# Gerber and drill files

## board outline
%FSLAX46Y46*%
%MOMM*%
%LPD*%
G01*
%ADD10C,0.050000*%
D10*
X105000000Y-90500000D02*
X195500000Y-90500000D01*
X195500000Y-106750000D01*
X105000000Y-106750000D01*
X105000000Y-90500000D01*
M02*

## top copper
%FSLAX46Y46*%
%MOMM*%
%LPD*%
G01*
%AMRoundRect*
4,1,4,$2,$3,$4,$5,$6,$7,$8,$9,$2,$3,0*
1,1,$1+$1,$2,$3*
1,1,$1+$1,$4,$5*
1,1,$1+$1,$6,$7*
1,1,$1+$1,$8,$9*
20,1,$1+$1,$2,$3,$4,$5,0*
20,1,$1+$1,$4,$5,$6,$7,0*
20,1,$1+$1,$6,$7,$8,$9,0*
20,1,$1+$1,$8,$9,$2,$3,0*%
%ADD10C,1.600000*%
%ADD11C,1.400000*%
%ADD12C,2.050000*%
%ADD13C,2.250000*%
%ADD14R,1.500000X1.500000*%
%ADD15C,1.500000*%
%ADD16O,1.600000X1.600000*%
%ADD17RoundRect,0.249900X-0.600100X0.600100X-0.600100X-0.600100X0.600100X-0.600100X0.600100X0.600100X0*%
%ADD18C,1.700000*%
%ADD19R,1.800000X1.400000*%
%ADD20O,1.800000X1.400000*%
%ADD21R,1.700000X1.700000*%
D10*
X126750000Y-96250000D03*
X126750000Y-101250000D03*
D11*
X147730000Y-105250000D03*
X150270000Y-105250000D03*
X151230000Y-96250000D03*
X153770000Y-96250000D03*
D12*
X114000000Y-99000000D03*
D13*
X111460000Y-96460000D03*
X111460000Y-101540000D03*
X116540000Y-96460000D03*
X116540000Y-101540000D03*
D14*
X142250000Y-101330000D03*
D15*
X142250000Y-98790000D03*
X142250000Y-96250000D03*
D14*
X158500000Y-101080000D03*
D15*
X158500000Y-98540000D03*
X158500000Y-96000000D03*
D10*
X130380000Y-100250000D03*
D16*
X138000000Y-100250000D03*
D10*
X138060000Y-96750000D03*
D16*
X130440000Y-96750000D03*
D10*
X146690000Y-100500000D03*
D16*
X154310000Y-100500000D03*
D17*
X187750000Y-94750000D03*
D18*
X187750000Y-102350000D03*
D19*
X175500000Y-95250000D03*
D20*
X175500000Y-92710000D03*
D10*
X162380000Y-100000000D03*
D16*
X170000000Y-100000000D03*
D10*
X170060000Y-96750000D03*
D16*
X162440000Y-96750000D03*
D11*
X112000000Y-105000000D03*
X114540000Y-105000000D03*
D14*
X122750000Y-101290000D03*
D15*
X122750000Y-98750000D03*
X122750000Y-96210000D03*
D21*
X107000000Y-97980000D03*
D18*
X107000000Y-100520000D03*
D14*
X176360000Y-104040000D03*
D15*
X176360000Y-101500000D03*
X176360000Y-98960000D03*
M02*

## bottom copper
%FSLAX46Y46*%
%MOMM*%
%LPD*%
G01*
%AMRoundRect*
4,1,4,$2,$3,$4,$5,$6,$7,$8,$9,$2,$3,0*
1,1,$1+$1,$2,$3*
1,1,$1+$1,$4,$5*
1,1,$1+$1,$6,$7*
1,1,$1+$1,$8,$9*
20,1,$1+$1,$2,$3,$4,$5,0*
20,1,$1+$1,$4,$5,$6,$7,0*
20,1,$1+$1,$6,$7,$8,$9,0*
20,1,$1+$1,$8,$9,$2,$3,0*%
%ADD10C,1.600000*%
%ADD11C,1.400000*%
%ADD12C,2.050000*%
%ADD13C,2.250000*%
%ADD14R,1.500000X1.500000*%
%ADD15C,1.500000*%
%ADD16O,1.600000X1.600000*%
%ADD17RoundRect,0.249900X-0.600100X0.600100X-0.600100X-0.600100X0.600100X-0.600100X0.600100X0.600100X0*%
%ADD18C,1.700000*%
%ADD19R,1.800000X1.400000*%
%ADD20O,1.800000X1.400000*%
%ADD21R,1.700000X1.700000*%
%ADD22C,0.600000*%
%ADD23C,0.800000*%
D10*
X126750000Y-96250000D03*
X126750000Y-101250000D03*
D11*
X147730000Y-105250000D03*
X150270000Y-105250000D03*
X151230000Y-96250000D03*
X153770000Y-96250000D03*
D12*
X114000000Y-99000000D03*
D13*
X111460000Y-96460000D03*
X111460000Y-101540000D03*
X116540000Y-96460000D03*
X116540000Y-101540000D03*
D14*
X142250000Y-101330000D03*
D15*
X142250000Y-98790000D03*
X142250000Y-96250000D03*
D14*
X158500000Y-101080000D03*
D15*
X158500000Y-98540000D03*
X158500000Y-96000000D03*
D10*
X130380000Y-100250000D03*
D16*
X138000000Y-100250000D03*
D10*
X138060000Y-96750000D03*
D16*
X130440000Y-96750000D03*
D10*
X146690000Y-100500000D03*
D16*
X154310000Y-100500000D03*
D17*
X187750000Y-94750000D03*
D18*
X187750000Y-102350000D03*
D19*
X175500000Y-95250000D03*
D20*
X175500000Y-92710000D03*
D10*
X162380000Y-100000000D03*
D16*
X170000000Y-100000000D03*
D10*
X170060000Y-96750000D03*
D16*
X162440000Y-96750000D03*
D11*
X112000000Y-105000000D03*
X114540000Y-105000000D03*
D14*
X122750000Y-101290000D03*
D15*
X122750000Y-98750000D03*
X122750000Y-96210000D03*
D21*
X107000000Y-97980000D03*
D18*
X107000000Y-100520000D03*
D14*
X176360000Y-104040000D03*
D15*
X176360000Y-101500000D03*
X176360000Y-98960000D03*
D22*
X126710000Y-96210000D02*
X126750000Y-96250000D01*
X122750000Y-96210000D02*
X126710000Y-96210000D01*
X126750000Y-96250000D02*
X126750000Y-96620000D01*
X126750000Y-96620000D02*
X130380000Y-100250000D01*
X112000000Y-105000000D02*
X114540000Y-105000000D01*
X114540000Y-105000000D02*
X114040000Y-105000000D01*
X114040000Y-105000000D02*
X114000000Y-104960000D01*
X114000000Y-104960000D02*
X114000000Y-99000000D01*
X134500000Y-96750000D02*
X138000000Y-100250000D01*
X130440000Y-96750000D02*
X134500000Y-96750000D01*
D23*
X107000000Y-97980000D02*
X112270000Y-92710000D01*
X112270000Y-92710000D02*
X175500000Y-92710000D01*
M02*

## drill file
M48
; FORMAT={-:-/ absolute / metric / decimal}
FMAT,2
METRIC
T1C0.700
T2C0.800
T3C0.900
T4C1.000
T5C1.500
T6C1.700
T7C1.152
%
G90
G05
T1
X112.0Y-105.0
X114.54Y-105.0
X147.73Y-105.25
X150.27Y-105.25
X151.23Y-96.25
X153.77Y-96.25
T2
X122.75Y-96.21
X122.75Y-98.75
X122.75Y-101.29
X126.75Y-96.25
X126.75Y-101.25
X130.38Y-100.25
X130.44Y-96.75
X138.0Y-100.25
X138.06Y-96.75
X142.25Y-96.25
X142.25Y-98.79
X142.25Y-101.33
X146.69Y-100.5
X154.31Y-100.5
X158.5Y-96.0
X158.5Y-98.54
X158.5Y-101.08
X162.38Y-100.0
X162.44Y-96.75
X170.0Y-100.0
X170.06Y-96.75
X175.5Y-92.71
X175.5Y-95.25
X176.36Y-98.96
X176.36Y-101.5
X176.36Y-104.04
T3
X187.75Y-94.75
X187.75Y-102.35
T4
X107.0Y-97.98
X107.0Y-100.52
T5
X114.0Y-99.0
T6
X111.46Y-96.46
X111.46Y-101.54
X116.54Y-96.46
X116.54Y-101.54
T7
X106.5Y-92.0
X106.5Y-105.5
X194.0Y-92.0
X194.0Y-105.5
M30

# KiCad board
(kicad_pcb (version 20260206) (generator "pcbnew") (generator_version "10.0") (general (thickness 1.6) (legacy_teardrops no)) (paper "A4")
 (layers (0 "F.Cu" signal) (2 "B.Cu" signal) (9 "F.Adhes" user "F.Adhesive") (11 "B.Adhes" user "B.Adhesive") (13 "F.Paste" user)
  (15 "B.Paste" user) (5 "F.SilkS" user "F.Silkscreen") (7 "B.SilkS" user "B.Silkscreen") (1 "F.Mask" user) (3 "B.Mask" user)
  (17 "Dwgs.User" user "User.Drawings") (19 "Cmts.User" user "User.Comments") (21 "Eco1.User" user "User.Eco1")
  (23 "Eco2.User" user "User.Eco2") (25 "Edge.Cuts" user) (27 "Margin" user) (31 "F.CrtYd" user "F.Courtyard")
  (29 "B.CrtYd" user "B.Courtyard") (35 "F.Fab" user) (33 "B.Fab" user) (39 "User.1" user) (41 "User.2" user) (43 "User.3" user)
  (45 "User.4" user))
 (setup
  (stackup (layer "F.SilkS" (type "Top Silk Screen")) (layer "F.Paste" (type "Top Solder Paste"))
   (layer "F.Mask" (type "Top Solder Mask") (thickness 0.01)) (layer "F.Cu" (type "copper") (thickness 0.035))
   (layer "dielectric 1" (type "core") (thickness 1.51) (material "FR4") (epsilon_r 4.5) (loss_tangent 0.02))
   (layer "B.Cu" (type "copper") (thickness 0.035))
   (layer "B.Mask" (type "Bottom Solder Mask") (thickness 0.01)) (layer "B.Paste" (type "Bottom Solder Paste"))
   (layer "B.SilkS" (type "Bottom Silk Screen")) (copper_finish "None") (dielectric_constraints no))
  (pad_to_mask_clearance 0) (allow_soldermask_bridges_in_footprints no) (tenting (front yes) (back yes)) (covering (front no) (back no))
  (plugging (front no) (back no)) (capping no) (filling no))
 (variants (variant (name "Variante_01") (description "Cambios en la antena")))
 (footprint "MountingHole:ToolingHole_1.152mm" (layer "F.Cu") (at 194 92)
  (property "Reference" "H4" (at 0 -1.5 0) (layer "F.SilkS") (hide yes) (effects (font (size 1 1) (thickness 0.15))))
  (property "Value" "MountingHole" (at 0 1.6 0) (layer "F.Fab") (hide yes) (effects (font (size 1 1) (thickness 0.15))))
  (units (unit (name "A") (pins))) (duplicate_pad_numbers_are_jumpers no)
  (pad "" np_thru_hole circle (at 0 0) (size 1.152 1.152) (drill 1.152) (layers "*.Cu" "*.Mask") (solder_mask_margin 0.074))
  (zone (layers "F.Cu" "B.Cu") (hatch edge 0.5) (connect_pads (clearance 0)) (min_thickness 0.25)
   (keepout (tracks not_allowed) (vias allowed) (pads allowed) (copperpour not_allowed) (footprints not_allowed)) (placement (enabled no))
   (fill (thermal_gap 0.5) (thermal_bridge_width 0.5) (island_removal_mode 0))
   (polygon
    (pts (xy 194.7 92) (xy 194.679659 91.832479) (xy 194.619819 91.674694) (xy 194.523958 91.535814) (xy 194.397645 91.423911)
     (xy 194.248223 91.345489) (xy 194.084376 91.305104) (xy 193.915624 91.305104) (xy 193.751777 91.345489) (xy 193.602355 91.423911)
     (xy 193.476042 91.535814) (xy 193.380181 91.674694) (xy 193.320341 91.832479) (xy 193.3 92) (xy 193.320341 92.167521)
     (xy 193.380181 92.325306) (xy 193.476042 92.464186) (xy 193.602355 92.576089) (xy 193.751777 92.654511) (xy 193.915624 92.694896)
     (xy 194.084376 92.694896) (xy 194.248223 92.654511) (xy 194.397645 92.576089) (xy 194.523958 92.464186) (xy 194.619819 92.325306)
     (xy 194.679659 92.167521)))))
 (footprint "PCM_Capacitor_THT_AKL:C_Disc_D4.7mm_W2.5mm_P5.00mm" (layer "F.Cu") (at 126.75 96.25 -90)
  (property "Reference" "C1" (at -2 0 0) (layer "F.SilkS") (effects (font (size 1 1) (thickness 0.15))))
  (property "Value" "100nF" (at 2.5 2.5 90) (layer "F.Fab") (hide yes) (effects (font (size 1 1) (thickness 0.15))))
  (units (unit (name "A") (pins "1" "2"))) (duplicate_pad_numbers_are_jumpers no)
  (pad "1" thru_hole circle (at 0 0 270) (size 1.6 1.6) (drill 0.8) (layers "*.Cu" "*.Mask") (remove_unused_layers no) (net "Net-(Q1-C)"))
  (pad "2" thru_hole circle (at 5 0 270) (size 1.6 1.6) (drill 0.8) (layers "*.Cu" "*.Mask") (remove_unused_layers no) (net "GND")))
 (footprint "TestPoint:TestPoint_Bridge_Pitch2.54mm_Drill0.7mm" (layer "F.Cu") (at 147.73 105.25)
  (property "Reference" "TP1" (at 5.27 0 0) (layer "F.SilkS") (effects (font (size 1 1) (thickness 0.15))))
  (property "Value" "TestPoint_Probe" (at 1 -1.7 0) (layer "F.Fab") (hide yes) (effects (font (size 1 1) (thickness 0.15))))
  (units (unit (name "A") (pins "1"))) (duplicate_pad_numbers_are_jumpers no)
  (pad "1" thru_hole circle (at 0 0) (size 1.4 1.4) (drill 0.7) (layers "*.Cu" "*.Mask") (remove_unused_layers no) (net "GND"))
  (pad "1" thru_hole circle (at 2.54 0) (size 1.4 1.4) (drill 0.7) (layers "*.Cu" "*.Mask") (remove_unused_layers no) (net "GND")))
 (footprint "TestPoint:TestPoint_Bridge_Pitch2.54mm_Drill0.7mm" (layer "F.Cu") (at 151.23 96.25)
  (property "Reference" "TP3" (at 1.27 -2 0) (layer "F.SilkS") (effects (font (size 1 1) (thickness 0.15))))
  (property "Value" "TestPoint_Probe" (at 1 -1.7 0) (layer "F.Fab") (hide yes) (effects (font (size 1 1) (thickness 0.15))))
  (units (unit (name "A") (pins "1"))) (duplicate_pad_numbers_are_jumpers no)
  (pad "1" thru_hole circle (at 0 0) (size 1.4 1.4) (drill 0.7) (layers "*.Cu" "*.Mask") (remove_unused_layers no) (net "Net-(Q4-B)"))
  (pad "1" thru_hole circle (at 2.54 0) (size 1.4 1.4) (drill 0.7) (layers "*.Cu" "*.Mask") (remove_unused_layers no) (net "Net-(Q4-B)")))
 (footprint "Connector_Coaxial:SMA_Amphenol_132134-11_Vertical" (layer "F.Cu") (at 114 99)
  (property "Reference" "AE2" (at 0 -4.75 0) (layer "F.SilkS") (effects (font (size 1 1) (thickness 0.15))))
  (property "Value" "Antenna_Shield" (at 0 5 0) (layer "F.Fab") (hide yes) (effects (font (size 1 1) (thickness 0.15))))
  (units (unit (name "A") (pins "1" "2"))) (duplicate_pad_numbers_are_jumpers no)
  (pad "1" thru_hole circle (at 0 0) (size 2.05 2.05) (drill 1.5) (layers "*.Cu" "*.Mask") (remove_unused_layers no) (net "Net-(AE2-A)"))
  (pad "2" thru_hole circle (at -2.54 -2.54) (size 2.25 2.25) (drill 1.7) (layers "*.Cu" "*.Mask") (remove_unused_layers no) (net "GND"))
  (pad "2" thru_hole circle (at -2.54 2.54) (size 2.25 2.25) (drill 1.7) (layers "*.Cu" "*.Mask") (remove_unused_layers no) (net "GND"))
  (pad "2" thru_hole circle (at 2.54 -2.54) (size 2.25 2.25) (drill 1.7) (layers "*.Cu" "*.Mask") (remove_unused_layers no) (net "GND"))
  (pad "2" thru_hole circle (at 2.54 2.54) (size 2.25 2.25) (drill 1.7) (layers "*.Cu" "*.Mask") (remove_unused_layers no) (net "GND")))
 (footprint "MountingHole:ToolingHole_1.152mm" (layer "F.Cu") (at 194 105.5)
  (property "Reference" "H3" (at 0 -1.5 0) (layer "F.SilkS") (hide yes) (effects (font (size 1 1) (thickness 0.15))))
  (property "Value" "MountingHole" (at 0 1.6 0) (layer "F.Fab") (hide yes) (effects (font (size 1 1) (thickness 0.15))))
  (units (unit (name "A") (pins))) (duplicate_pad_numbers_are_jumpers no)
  (pad "" np_thru_hole circle (at 0 0) (size 1.152 1.152) (drill 1.152) (layers "*.Cu" "*.Mask") (solder_mask_margin 0.074))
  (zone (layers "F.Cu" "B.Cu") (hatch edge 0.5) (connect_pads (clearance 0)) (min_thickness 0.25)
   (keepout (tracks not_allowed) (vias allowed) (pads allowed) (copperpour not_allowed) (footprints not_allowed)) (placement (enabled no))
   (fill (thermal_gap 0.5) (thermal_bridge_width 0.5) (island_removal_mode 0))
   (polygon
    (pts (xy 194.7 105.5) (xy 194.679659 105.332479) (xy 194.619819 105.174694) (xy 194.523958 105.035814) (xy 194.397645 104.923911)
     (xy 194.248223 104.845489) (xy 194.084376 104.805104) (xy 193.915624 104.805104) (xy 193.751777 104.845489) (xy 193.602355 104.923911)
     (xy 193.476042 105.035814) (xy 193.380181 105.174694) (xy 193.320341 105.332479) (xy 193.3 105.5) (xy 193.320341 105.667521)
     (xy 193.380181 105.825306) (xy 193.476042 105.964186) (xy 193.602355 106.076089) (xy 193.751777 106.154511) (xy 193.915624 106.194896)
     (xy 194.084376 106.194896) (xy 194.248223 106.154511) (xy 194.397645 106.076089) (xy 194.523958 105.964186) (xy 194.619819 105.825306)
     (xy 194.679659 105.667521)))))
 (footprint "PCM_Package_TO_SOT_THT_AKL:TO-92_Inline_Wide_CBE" (layer "F.Cu") (at 142.25 101.33 90)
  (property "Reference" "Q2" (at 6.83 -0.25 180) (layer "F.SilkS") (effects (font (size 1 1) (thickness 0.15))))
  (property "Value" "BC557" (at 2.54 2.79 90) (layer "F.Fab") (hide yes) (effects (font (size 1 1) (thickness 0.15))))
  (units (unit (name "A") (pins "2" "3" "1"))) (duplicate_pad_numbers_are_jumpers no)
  (pad "1" thru_hole rect (at 0 0 180) (size 1.5 1.5) (drill 0.8) (layers "*.Cu" "*.Mask") (remove_unused_layers no) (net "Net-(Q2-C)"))
  (pad "2" thru_hole circle (at 2.54 0 180) (size 1.5 1.5) (drill 0.8) (layers "*.Cu" "*.Mask") (remove_unused_layers no) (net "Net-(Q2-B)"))
  (pad "3" thru_hole circle (at 5.08 0 180) (size 1.5 1.5) (drill 0.8) (layers "*.Cu" "*.Mask") (remove_unused_layers no) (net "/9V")))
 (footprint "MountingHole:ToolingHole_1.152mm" (layer "F.Cu") (at 106.5 92)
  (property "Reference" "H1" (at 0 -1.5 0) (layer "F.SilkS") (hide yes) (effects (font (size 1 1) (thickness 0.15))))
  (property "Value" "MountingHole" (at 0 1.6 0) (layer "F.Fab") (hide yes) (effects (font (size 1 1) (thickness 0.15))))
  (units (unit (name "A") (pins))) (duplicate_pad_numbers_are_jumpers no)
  (pad "" np_thru_hole circle (at 0 0) (size 1.152 1.152) (drill 1.152) (layers "*.Cu" "*.Mask") (solder_mask_margin 0.074))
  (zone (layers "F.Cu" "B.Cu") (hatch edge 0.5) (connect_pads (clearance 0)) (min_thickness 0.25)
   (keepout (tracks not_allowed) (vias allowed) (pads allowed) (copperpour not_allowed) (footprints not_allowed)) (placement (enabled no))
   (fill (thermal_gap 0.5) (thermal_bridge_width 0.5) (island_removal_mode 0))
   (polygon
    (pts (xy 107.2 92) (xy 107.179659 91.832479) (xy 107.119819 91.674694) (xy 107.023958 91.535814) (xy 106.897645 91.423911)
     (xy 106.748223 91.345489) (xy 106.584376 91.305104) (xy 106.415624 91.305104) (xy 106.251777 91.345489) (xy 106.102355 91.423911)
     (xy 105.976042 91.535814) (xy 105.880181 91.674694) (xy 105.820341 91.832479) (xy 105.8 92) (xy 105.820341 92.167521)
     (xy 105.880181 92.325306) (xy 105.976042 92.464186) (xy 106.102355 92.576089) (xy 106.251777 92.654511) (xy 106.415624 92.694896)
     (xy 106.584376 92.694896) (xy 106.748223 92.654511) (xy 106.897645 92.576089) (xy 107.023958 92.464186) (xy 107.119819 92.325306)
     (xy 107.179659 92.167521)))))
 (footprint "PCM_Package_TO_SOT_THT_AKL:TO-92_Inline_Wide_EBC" (layer "F.Cu") (at 158.5 101.08 90)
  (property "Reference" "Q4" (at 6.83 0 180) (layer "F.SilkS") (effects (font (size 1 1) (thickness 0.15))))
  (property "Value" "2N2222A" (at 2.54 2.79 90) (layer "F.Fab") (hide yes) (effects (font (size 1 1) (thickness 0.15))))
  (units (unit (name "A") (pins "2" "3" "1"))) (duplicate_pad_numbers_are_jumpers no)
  (pad "1" thru_hole rect (at 0 0 180) (size 1.5 1.5) (drill 0.8) (layers "*.Cu" "*.Mask") (remove_unused_layers no) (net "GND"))
  (pad "2" thru_hole circle (at 2.54 0 180) (size 1.5 1.5) (drill 0.8) (layers "*.Cu" "*.Mask") (remove_unused_layers no) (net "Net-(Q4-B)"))
  (pad "3" thru_hole circle (at 5.08 0 180) (size 1.5 1.5) (drill 0.8) (layers "*.Cu" "*.Mask") (remove_unused_layers no) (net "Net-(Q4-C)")))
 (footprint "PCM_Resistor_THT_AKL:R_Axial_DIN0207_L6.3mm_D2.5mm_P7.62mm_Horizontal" (layer "F.Cu") (at 130.38 100.25)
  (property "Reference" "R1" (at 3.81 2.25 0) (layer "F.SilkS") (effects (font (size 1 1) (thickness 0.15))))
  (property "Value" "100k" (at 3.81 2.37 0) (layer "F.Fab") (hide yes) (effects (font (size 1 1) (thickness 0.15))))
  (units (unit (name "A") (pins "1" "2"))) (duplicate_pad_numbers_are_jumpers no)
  (pad "1" thru_hole circle (at 0 0) (size 1.6 1.6) (drill 0.8) (layers "*.Cu" "*.Mask") (remove_unused_layers no) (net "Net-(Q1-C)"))
  (pad "2" thru_hole oval (at 7.62 0) (size 1.6 1.6) (drill 0.8) (layers "*.Cu" "*.Mask") (remove_unused_layers no) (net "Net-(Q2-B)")))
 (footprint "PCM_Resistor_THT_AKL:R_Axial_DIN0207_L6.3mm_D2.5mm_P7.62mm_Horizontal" (layer "F.Cu") (at 138.06 96.75 180)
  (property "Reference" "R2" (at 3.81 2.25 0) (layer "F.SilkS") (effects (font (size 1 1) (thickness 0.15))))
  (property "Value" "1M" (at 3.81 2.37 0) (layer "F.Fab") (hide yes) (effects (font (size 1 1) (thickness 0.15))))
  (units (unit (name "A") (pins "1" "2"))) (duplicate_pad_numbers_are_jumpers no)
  (pad "1" thru_hole circle (at 0 0 180) (size 1.6 1.6) (drill 0.8) (layers "*.Cu" "*.Mask") (remove_unused_layers no) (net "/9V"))
  (pad "2" thru_hole oval (at 7.62 0 180) (size 1.6 1.6) (drill 0.8) (layers "*.Cu" "*.Mask") (remove_unused_layers no) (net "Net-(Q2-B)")))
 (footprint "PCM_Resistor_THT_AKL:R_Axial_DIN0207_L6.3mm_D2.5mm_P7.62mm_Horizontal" (layer "F.Cu") (at 146.69 100.5)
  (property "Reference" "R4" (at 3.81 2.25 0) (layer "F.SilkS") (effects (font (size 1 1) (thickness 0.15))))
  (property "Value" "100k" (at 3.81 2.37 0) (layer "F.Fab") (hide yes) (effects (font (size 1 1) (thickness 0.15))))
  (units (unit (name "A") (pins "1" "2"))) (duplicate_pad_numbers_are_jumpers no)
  (pad "1" thru_hole circle (at 0 0) (size 1.6 1.6) (drill 0.8) (layers "*.Cu" "*.Mask") (remove_unused_layers no) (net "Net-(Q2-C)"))
  (pad "2" thru_hole oval (at 7.62 0) (size 1.6 1.6) (drill 0.8) (layers "*.Cu" "*.Mask") (remove_unused_layers no) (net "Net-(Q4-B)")))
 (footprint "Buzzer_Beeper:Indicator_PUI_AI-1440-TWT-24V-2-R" (layer "F.Cu") (at 187.75 94.75 -90)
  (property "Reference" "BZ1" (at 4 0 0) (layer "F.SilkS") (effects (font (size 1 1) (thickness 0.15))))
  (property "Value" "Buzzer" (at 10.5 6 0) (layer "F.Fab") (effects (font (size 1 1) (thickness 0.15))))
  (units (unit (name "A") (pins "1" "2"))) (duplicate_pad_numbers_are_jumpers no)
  (pad "1" thru_hole roundrect (at 0 0 270) (size 1.7 1.7) (drill 0.9) (layers "*.Cu" "*.Mask") (remove_unused_layers no)
   (roundrect_rratio 0.147) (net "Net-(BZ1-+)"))
  (pad "2" thru_hole circle (at 7.6 0 270) (size 1.7 1.7) (drill 0.9) (layers "*.Cu" "*.Mask") (remove_unused_layers no) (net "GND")))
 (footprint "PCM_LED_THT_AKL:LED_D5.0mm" (layer "F.Cu") (at 175.5 95.25 90)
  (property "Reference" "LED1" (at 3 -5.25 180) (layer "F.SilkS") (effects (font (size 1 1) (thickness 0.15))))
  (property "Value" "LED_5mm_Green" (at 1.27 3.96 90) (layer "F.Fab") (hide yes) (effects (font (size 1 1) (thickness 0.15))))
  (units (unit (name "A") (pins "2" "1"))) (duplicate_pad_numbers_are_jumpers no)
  (pad "1" thru_hole rect (at 0 0 90) (size 1.4 1.8) (drill 0.8) (layers "*.Cu" "*.Mask") (remove_unused_layers no) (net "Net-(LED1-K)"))
  (pad "2" thru_hole oval (at 2.54 0 90) (size 1.4 1.8) (drill 0.8) (layers "*.Cu" "*.Mask") (remove_unused_layers no) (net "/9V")))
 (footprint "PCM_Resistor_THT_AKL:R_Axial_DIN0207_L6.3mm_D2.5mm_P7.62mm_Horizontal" (layer "F.Cu") (at 162.38 100)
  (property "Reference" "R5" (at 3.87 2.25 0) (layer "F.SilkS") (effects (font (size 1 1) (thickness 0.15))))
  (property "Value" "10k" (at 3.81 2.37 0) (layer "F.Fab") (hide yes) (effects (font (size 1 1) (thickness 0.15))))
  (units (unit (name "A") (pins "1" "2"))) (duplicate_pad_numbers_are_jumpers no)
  (pad "1" thru_hole circle (at 0 0) (size 1.6 1.6) (drill 0.8) (layers "*.Cu" "*.Mask") (remove_unused_layers no) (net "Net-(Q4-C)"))
  (pad "2" thru_hole oval (at 7.62 0) (size 1.6 1.6) (drill 0.8) (layers "*.Cu" "*.Mask") (remove_unused_layers no) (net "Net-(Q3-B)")))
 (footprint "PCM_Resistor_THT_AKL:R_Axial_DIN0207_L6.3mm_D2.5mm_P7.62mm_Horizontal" (layer "F.Cu") (at 170.06 96.75 180)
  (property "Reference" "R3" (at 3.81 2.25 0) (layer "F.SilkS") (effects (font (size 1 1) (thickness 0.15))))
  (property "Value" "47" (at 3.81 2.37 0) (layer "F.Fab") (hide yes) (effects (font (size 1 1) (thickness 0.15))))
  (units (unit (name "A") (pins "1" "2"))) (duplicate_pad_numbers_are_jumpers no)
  (pad "1" thru_hole circle (at 0 0 180) (size 1.6 1.6) (drill 0.8) (layers "*.Cu" "*.Mask") (remove_unused_layers no) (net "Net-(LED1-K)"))
  (pad "2" thru_hole oval (at 7.62 0 180) (size 1.6 1.6) (drill 0.8) (layers "*.Cu" "*.Mask") (remove_unused_layers no) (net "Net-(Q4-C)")))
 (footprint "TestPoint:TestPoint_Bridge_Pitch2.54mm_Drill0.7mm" (layer "F.Cu") (at 112 105)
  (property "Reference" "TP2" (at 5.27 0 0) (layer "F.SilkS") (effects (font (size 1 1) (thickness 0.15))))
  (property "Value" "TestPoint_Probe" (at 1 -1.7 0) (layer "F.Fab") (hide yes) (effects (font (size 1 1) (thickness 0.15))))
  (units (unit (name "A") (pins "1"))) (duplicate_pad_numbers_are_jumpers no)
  (pad "1" thru_hole circle (at 0 0) (size 1.4 1.4) (drill 0.7) (layers "*.Cu" "*.Mask") (remove_unused_layers no) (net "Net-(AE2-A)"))
  (pad "1" thru_hole circle (at 2.54 0) (size 1.4 1.4) (drill 0.7) (layers "*.Cu" "*.Mask") (remove_unused_layers no) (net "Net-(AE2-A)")))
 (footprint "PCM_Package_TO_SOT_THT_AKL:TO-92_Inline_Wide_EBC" (layer "F.Cu") (at 122.75 101.29 90)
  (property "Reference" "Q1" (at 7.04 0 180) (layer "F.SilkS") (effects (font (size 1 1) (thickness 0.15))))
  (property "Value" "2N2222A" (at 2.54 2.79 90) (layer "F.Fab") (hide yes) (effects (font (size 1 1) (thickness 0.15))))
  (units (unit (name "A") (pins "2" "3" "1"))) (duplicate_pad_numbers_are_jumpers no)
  (pad "1" thru_hole rect (at 0 0 180) (size 1.5 1.5) (drill 0.8) (layers "*.Cu" "*.Mask") (remove_unused_layers no) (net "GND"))
  (pad "2" thru_hole circle (at 2.54 0 180) (size 1.5 1.5) (drill 0.8) (layers "*.Cu" "*.Mask") (remove_unused_layers no)
   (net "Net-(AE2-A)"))
  (pad "3" thru_hole circle (at 5.08 0 180) (size 1.5 1.5) (drill 0.8) (layers "*.Cu" "*.Mask") (remove_unused_layers no) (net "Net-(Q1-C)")))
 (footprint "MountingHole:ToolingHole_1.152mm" (layer "F.Cu") (at 106.5 105.5)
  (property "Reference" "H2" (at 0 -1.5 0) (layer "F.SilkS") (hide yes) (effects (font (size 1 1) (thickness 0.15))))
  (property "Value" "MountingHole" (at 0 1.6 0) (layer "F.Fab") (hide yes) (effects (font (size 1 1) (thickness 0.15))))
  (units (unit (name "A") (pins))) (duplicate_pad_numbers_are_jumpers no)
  (pad "" np_thru_hole circle (at 0 0) (size 1.152 1.152) (drill 1.152) (layers "*.Cu" "*.Mask") (solder_mask_margin 0.074))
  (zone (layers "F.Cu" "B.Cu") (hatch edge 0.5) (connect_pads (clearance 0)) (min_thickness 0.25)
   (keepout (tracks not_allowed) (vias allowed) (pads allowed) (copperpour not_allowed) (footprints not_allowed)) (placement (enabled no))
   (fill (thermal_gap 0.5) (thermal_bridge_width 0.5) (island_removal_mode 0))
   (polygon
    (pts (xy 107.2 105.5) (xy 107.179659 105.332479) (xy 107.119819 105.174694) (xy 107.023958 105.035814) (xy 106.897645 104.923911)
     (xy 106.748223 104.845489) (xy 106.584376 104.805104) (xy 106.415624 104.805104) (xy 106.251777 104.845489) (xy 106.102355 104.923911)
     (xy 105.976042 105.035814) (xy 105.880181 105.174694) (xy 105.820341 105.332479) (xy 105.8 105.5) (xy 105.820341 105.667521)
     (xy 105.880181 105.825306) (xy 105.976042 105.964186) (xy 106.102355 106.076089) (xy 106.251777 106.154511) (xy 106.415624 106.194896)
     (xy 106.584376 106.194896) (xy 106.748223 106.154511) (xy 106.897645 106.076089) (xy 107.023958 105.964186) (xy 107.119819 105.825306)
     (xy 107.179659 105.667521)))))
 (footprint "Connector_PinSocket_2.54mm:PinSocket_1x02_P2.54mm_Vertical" (layer "F.Cu") (at 107 97.98)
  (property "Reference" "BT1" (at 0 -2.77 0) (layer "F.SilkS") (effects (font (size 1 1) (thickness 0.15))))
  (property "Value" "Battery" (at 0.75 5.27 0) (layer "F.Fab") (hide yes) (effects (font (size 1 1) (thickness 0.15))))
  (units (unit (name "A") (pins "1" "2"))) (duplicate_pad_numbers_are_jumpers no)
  (pad "1" thru_hole rect (at 0 0) (size 1.7 1.7) (drill 1) (layers "*.Cu" "*.Mask") (remove_unused_layers no) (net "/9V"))
  (pad "2" thru_hole circle (at 0 2.54) (size 1.7 1.7) (drill 1) (layers "*.Cu" "*.Mask") (remove_unused_layers no) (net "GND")))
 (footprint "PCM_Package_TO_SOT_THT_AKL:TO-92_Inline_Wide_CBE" (layer "F.Cu") (at 176.36 104.04 90)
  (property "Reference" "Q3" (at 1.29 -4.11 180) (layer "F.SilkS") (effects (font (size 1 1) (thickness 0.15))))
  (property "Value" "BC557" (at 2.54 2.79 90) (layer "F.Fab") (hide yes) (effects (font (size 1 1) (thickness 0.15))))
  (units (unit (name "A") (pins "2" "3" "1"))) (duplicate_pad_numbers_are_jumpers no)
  (pad "1" thru_hole rect (at 0 0 180) (size 1.5 1.5) (drill 0.8) (layers "*.Cu" "*.Mask") (remove_unused_layers no) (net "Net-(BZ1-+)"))
  (pad "2" thru_hole circle (at 2.54 0 180) (size 1.5 1.5) (drill 0.8) (layers "*.Cu" "*.Mask") (remove_unused_layers no) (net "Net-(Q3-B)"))
  (pad "3" thru_hole circle (at 5.08 0 180) (size 1.5 1.5) (drill 0.8) (layers "*.Cu" "*.Mask") (remove_unused_layers no) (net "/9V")))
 (gr_rect (start 105 90.5) (end 195.5 106.75) (stroke (width 0.05) (type default)) (fill no) (layer "Edge.Cuts"))
 (segment (start 126.71 96.21) (end 126.75 96.25) (width 0.6) (layer "B.Cu") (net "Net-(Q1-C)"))
 (segment (start 122.75 96.21) (end 126.71 96.21) (width 0.6) (layer "B.Cu") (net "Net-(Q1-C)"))
 (segment (start 126.75 96.25) (end 126.75 96.62) (width 0.6) (layer "B.Cu") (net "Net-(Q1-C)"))
 (segment (start 126.75 96.62) (end 130.38 100.25) (width 0.6) (layer "B.Cu") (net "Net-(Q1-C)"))
 (segment (start 112 105) (end 114.54 105) (width 0.6) (layer "B.Cu") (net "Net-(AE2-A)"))
 (segment (start 114.54 105) (end 114.04 105) (width 0.6) (layer "B.Cu") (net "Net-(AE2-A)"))
 (segment (start 114.04 105) (end 114 104.96) (width 0.6) (layer "B.Cu") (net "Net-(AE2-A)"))
 (segment (start 114 104.96) (end 114 99) (width 0.6) (layer "B.Cu") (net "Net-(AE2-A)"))
 (segment (start 134.5 96.75) (end 138 100.25) (width 0.6) (layer "B.Cu") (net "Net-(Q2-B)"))
 (segment (start 130.44 96.75) (end 134.5 96.75) (width 0.6) (layer "B.Cu") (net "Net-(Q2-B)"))
 (segment (start 107 97.98) (end 112.27 92.71) (width 0.8) (layer "B.Cu") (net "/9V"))
 (segment (start 112.27 92.71) (end 175.5 92.71) (width 0.8) (layer "B.Cu") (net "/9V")))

